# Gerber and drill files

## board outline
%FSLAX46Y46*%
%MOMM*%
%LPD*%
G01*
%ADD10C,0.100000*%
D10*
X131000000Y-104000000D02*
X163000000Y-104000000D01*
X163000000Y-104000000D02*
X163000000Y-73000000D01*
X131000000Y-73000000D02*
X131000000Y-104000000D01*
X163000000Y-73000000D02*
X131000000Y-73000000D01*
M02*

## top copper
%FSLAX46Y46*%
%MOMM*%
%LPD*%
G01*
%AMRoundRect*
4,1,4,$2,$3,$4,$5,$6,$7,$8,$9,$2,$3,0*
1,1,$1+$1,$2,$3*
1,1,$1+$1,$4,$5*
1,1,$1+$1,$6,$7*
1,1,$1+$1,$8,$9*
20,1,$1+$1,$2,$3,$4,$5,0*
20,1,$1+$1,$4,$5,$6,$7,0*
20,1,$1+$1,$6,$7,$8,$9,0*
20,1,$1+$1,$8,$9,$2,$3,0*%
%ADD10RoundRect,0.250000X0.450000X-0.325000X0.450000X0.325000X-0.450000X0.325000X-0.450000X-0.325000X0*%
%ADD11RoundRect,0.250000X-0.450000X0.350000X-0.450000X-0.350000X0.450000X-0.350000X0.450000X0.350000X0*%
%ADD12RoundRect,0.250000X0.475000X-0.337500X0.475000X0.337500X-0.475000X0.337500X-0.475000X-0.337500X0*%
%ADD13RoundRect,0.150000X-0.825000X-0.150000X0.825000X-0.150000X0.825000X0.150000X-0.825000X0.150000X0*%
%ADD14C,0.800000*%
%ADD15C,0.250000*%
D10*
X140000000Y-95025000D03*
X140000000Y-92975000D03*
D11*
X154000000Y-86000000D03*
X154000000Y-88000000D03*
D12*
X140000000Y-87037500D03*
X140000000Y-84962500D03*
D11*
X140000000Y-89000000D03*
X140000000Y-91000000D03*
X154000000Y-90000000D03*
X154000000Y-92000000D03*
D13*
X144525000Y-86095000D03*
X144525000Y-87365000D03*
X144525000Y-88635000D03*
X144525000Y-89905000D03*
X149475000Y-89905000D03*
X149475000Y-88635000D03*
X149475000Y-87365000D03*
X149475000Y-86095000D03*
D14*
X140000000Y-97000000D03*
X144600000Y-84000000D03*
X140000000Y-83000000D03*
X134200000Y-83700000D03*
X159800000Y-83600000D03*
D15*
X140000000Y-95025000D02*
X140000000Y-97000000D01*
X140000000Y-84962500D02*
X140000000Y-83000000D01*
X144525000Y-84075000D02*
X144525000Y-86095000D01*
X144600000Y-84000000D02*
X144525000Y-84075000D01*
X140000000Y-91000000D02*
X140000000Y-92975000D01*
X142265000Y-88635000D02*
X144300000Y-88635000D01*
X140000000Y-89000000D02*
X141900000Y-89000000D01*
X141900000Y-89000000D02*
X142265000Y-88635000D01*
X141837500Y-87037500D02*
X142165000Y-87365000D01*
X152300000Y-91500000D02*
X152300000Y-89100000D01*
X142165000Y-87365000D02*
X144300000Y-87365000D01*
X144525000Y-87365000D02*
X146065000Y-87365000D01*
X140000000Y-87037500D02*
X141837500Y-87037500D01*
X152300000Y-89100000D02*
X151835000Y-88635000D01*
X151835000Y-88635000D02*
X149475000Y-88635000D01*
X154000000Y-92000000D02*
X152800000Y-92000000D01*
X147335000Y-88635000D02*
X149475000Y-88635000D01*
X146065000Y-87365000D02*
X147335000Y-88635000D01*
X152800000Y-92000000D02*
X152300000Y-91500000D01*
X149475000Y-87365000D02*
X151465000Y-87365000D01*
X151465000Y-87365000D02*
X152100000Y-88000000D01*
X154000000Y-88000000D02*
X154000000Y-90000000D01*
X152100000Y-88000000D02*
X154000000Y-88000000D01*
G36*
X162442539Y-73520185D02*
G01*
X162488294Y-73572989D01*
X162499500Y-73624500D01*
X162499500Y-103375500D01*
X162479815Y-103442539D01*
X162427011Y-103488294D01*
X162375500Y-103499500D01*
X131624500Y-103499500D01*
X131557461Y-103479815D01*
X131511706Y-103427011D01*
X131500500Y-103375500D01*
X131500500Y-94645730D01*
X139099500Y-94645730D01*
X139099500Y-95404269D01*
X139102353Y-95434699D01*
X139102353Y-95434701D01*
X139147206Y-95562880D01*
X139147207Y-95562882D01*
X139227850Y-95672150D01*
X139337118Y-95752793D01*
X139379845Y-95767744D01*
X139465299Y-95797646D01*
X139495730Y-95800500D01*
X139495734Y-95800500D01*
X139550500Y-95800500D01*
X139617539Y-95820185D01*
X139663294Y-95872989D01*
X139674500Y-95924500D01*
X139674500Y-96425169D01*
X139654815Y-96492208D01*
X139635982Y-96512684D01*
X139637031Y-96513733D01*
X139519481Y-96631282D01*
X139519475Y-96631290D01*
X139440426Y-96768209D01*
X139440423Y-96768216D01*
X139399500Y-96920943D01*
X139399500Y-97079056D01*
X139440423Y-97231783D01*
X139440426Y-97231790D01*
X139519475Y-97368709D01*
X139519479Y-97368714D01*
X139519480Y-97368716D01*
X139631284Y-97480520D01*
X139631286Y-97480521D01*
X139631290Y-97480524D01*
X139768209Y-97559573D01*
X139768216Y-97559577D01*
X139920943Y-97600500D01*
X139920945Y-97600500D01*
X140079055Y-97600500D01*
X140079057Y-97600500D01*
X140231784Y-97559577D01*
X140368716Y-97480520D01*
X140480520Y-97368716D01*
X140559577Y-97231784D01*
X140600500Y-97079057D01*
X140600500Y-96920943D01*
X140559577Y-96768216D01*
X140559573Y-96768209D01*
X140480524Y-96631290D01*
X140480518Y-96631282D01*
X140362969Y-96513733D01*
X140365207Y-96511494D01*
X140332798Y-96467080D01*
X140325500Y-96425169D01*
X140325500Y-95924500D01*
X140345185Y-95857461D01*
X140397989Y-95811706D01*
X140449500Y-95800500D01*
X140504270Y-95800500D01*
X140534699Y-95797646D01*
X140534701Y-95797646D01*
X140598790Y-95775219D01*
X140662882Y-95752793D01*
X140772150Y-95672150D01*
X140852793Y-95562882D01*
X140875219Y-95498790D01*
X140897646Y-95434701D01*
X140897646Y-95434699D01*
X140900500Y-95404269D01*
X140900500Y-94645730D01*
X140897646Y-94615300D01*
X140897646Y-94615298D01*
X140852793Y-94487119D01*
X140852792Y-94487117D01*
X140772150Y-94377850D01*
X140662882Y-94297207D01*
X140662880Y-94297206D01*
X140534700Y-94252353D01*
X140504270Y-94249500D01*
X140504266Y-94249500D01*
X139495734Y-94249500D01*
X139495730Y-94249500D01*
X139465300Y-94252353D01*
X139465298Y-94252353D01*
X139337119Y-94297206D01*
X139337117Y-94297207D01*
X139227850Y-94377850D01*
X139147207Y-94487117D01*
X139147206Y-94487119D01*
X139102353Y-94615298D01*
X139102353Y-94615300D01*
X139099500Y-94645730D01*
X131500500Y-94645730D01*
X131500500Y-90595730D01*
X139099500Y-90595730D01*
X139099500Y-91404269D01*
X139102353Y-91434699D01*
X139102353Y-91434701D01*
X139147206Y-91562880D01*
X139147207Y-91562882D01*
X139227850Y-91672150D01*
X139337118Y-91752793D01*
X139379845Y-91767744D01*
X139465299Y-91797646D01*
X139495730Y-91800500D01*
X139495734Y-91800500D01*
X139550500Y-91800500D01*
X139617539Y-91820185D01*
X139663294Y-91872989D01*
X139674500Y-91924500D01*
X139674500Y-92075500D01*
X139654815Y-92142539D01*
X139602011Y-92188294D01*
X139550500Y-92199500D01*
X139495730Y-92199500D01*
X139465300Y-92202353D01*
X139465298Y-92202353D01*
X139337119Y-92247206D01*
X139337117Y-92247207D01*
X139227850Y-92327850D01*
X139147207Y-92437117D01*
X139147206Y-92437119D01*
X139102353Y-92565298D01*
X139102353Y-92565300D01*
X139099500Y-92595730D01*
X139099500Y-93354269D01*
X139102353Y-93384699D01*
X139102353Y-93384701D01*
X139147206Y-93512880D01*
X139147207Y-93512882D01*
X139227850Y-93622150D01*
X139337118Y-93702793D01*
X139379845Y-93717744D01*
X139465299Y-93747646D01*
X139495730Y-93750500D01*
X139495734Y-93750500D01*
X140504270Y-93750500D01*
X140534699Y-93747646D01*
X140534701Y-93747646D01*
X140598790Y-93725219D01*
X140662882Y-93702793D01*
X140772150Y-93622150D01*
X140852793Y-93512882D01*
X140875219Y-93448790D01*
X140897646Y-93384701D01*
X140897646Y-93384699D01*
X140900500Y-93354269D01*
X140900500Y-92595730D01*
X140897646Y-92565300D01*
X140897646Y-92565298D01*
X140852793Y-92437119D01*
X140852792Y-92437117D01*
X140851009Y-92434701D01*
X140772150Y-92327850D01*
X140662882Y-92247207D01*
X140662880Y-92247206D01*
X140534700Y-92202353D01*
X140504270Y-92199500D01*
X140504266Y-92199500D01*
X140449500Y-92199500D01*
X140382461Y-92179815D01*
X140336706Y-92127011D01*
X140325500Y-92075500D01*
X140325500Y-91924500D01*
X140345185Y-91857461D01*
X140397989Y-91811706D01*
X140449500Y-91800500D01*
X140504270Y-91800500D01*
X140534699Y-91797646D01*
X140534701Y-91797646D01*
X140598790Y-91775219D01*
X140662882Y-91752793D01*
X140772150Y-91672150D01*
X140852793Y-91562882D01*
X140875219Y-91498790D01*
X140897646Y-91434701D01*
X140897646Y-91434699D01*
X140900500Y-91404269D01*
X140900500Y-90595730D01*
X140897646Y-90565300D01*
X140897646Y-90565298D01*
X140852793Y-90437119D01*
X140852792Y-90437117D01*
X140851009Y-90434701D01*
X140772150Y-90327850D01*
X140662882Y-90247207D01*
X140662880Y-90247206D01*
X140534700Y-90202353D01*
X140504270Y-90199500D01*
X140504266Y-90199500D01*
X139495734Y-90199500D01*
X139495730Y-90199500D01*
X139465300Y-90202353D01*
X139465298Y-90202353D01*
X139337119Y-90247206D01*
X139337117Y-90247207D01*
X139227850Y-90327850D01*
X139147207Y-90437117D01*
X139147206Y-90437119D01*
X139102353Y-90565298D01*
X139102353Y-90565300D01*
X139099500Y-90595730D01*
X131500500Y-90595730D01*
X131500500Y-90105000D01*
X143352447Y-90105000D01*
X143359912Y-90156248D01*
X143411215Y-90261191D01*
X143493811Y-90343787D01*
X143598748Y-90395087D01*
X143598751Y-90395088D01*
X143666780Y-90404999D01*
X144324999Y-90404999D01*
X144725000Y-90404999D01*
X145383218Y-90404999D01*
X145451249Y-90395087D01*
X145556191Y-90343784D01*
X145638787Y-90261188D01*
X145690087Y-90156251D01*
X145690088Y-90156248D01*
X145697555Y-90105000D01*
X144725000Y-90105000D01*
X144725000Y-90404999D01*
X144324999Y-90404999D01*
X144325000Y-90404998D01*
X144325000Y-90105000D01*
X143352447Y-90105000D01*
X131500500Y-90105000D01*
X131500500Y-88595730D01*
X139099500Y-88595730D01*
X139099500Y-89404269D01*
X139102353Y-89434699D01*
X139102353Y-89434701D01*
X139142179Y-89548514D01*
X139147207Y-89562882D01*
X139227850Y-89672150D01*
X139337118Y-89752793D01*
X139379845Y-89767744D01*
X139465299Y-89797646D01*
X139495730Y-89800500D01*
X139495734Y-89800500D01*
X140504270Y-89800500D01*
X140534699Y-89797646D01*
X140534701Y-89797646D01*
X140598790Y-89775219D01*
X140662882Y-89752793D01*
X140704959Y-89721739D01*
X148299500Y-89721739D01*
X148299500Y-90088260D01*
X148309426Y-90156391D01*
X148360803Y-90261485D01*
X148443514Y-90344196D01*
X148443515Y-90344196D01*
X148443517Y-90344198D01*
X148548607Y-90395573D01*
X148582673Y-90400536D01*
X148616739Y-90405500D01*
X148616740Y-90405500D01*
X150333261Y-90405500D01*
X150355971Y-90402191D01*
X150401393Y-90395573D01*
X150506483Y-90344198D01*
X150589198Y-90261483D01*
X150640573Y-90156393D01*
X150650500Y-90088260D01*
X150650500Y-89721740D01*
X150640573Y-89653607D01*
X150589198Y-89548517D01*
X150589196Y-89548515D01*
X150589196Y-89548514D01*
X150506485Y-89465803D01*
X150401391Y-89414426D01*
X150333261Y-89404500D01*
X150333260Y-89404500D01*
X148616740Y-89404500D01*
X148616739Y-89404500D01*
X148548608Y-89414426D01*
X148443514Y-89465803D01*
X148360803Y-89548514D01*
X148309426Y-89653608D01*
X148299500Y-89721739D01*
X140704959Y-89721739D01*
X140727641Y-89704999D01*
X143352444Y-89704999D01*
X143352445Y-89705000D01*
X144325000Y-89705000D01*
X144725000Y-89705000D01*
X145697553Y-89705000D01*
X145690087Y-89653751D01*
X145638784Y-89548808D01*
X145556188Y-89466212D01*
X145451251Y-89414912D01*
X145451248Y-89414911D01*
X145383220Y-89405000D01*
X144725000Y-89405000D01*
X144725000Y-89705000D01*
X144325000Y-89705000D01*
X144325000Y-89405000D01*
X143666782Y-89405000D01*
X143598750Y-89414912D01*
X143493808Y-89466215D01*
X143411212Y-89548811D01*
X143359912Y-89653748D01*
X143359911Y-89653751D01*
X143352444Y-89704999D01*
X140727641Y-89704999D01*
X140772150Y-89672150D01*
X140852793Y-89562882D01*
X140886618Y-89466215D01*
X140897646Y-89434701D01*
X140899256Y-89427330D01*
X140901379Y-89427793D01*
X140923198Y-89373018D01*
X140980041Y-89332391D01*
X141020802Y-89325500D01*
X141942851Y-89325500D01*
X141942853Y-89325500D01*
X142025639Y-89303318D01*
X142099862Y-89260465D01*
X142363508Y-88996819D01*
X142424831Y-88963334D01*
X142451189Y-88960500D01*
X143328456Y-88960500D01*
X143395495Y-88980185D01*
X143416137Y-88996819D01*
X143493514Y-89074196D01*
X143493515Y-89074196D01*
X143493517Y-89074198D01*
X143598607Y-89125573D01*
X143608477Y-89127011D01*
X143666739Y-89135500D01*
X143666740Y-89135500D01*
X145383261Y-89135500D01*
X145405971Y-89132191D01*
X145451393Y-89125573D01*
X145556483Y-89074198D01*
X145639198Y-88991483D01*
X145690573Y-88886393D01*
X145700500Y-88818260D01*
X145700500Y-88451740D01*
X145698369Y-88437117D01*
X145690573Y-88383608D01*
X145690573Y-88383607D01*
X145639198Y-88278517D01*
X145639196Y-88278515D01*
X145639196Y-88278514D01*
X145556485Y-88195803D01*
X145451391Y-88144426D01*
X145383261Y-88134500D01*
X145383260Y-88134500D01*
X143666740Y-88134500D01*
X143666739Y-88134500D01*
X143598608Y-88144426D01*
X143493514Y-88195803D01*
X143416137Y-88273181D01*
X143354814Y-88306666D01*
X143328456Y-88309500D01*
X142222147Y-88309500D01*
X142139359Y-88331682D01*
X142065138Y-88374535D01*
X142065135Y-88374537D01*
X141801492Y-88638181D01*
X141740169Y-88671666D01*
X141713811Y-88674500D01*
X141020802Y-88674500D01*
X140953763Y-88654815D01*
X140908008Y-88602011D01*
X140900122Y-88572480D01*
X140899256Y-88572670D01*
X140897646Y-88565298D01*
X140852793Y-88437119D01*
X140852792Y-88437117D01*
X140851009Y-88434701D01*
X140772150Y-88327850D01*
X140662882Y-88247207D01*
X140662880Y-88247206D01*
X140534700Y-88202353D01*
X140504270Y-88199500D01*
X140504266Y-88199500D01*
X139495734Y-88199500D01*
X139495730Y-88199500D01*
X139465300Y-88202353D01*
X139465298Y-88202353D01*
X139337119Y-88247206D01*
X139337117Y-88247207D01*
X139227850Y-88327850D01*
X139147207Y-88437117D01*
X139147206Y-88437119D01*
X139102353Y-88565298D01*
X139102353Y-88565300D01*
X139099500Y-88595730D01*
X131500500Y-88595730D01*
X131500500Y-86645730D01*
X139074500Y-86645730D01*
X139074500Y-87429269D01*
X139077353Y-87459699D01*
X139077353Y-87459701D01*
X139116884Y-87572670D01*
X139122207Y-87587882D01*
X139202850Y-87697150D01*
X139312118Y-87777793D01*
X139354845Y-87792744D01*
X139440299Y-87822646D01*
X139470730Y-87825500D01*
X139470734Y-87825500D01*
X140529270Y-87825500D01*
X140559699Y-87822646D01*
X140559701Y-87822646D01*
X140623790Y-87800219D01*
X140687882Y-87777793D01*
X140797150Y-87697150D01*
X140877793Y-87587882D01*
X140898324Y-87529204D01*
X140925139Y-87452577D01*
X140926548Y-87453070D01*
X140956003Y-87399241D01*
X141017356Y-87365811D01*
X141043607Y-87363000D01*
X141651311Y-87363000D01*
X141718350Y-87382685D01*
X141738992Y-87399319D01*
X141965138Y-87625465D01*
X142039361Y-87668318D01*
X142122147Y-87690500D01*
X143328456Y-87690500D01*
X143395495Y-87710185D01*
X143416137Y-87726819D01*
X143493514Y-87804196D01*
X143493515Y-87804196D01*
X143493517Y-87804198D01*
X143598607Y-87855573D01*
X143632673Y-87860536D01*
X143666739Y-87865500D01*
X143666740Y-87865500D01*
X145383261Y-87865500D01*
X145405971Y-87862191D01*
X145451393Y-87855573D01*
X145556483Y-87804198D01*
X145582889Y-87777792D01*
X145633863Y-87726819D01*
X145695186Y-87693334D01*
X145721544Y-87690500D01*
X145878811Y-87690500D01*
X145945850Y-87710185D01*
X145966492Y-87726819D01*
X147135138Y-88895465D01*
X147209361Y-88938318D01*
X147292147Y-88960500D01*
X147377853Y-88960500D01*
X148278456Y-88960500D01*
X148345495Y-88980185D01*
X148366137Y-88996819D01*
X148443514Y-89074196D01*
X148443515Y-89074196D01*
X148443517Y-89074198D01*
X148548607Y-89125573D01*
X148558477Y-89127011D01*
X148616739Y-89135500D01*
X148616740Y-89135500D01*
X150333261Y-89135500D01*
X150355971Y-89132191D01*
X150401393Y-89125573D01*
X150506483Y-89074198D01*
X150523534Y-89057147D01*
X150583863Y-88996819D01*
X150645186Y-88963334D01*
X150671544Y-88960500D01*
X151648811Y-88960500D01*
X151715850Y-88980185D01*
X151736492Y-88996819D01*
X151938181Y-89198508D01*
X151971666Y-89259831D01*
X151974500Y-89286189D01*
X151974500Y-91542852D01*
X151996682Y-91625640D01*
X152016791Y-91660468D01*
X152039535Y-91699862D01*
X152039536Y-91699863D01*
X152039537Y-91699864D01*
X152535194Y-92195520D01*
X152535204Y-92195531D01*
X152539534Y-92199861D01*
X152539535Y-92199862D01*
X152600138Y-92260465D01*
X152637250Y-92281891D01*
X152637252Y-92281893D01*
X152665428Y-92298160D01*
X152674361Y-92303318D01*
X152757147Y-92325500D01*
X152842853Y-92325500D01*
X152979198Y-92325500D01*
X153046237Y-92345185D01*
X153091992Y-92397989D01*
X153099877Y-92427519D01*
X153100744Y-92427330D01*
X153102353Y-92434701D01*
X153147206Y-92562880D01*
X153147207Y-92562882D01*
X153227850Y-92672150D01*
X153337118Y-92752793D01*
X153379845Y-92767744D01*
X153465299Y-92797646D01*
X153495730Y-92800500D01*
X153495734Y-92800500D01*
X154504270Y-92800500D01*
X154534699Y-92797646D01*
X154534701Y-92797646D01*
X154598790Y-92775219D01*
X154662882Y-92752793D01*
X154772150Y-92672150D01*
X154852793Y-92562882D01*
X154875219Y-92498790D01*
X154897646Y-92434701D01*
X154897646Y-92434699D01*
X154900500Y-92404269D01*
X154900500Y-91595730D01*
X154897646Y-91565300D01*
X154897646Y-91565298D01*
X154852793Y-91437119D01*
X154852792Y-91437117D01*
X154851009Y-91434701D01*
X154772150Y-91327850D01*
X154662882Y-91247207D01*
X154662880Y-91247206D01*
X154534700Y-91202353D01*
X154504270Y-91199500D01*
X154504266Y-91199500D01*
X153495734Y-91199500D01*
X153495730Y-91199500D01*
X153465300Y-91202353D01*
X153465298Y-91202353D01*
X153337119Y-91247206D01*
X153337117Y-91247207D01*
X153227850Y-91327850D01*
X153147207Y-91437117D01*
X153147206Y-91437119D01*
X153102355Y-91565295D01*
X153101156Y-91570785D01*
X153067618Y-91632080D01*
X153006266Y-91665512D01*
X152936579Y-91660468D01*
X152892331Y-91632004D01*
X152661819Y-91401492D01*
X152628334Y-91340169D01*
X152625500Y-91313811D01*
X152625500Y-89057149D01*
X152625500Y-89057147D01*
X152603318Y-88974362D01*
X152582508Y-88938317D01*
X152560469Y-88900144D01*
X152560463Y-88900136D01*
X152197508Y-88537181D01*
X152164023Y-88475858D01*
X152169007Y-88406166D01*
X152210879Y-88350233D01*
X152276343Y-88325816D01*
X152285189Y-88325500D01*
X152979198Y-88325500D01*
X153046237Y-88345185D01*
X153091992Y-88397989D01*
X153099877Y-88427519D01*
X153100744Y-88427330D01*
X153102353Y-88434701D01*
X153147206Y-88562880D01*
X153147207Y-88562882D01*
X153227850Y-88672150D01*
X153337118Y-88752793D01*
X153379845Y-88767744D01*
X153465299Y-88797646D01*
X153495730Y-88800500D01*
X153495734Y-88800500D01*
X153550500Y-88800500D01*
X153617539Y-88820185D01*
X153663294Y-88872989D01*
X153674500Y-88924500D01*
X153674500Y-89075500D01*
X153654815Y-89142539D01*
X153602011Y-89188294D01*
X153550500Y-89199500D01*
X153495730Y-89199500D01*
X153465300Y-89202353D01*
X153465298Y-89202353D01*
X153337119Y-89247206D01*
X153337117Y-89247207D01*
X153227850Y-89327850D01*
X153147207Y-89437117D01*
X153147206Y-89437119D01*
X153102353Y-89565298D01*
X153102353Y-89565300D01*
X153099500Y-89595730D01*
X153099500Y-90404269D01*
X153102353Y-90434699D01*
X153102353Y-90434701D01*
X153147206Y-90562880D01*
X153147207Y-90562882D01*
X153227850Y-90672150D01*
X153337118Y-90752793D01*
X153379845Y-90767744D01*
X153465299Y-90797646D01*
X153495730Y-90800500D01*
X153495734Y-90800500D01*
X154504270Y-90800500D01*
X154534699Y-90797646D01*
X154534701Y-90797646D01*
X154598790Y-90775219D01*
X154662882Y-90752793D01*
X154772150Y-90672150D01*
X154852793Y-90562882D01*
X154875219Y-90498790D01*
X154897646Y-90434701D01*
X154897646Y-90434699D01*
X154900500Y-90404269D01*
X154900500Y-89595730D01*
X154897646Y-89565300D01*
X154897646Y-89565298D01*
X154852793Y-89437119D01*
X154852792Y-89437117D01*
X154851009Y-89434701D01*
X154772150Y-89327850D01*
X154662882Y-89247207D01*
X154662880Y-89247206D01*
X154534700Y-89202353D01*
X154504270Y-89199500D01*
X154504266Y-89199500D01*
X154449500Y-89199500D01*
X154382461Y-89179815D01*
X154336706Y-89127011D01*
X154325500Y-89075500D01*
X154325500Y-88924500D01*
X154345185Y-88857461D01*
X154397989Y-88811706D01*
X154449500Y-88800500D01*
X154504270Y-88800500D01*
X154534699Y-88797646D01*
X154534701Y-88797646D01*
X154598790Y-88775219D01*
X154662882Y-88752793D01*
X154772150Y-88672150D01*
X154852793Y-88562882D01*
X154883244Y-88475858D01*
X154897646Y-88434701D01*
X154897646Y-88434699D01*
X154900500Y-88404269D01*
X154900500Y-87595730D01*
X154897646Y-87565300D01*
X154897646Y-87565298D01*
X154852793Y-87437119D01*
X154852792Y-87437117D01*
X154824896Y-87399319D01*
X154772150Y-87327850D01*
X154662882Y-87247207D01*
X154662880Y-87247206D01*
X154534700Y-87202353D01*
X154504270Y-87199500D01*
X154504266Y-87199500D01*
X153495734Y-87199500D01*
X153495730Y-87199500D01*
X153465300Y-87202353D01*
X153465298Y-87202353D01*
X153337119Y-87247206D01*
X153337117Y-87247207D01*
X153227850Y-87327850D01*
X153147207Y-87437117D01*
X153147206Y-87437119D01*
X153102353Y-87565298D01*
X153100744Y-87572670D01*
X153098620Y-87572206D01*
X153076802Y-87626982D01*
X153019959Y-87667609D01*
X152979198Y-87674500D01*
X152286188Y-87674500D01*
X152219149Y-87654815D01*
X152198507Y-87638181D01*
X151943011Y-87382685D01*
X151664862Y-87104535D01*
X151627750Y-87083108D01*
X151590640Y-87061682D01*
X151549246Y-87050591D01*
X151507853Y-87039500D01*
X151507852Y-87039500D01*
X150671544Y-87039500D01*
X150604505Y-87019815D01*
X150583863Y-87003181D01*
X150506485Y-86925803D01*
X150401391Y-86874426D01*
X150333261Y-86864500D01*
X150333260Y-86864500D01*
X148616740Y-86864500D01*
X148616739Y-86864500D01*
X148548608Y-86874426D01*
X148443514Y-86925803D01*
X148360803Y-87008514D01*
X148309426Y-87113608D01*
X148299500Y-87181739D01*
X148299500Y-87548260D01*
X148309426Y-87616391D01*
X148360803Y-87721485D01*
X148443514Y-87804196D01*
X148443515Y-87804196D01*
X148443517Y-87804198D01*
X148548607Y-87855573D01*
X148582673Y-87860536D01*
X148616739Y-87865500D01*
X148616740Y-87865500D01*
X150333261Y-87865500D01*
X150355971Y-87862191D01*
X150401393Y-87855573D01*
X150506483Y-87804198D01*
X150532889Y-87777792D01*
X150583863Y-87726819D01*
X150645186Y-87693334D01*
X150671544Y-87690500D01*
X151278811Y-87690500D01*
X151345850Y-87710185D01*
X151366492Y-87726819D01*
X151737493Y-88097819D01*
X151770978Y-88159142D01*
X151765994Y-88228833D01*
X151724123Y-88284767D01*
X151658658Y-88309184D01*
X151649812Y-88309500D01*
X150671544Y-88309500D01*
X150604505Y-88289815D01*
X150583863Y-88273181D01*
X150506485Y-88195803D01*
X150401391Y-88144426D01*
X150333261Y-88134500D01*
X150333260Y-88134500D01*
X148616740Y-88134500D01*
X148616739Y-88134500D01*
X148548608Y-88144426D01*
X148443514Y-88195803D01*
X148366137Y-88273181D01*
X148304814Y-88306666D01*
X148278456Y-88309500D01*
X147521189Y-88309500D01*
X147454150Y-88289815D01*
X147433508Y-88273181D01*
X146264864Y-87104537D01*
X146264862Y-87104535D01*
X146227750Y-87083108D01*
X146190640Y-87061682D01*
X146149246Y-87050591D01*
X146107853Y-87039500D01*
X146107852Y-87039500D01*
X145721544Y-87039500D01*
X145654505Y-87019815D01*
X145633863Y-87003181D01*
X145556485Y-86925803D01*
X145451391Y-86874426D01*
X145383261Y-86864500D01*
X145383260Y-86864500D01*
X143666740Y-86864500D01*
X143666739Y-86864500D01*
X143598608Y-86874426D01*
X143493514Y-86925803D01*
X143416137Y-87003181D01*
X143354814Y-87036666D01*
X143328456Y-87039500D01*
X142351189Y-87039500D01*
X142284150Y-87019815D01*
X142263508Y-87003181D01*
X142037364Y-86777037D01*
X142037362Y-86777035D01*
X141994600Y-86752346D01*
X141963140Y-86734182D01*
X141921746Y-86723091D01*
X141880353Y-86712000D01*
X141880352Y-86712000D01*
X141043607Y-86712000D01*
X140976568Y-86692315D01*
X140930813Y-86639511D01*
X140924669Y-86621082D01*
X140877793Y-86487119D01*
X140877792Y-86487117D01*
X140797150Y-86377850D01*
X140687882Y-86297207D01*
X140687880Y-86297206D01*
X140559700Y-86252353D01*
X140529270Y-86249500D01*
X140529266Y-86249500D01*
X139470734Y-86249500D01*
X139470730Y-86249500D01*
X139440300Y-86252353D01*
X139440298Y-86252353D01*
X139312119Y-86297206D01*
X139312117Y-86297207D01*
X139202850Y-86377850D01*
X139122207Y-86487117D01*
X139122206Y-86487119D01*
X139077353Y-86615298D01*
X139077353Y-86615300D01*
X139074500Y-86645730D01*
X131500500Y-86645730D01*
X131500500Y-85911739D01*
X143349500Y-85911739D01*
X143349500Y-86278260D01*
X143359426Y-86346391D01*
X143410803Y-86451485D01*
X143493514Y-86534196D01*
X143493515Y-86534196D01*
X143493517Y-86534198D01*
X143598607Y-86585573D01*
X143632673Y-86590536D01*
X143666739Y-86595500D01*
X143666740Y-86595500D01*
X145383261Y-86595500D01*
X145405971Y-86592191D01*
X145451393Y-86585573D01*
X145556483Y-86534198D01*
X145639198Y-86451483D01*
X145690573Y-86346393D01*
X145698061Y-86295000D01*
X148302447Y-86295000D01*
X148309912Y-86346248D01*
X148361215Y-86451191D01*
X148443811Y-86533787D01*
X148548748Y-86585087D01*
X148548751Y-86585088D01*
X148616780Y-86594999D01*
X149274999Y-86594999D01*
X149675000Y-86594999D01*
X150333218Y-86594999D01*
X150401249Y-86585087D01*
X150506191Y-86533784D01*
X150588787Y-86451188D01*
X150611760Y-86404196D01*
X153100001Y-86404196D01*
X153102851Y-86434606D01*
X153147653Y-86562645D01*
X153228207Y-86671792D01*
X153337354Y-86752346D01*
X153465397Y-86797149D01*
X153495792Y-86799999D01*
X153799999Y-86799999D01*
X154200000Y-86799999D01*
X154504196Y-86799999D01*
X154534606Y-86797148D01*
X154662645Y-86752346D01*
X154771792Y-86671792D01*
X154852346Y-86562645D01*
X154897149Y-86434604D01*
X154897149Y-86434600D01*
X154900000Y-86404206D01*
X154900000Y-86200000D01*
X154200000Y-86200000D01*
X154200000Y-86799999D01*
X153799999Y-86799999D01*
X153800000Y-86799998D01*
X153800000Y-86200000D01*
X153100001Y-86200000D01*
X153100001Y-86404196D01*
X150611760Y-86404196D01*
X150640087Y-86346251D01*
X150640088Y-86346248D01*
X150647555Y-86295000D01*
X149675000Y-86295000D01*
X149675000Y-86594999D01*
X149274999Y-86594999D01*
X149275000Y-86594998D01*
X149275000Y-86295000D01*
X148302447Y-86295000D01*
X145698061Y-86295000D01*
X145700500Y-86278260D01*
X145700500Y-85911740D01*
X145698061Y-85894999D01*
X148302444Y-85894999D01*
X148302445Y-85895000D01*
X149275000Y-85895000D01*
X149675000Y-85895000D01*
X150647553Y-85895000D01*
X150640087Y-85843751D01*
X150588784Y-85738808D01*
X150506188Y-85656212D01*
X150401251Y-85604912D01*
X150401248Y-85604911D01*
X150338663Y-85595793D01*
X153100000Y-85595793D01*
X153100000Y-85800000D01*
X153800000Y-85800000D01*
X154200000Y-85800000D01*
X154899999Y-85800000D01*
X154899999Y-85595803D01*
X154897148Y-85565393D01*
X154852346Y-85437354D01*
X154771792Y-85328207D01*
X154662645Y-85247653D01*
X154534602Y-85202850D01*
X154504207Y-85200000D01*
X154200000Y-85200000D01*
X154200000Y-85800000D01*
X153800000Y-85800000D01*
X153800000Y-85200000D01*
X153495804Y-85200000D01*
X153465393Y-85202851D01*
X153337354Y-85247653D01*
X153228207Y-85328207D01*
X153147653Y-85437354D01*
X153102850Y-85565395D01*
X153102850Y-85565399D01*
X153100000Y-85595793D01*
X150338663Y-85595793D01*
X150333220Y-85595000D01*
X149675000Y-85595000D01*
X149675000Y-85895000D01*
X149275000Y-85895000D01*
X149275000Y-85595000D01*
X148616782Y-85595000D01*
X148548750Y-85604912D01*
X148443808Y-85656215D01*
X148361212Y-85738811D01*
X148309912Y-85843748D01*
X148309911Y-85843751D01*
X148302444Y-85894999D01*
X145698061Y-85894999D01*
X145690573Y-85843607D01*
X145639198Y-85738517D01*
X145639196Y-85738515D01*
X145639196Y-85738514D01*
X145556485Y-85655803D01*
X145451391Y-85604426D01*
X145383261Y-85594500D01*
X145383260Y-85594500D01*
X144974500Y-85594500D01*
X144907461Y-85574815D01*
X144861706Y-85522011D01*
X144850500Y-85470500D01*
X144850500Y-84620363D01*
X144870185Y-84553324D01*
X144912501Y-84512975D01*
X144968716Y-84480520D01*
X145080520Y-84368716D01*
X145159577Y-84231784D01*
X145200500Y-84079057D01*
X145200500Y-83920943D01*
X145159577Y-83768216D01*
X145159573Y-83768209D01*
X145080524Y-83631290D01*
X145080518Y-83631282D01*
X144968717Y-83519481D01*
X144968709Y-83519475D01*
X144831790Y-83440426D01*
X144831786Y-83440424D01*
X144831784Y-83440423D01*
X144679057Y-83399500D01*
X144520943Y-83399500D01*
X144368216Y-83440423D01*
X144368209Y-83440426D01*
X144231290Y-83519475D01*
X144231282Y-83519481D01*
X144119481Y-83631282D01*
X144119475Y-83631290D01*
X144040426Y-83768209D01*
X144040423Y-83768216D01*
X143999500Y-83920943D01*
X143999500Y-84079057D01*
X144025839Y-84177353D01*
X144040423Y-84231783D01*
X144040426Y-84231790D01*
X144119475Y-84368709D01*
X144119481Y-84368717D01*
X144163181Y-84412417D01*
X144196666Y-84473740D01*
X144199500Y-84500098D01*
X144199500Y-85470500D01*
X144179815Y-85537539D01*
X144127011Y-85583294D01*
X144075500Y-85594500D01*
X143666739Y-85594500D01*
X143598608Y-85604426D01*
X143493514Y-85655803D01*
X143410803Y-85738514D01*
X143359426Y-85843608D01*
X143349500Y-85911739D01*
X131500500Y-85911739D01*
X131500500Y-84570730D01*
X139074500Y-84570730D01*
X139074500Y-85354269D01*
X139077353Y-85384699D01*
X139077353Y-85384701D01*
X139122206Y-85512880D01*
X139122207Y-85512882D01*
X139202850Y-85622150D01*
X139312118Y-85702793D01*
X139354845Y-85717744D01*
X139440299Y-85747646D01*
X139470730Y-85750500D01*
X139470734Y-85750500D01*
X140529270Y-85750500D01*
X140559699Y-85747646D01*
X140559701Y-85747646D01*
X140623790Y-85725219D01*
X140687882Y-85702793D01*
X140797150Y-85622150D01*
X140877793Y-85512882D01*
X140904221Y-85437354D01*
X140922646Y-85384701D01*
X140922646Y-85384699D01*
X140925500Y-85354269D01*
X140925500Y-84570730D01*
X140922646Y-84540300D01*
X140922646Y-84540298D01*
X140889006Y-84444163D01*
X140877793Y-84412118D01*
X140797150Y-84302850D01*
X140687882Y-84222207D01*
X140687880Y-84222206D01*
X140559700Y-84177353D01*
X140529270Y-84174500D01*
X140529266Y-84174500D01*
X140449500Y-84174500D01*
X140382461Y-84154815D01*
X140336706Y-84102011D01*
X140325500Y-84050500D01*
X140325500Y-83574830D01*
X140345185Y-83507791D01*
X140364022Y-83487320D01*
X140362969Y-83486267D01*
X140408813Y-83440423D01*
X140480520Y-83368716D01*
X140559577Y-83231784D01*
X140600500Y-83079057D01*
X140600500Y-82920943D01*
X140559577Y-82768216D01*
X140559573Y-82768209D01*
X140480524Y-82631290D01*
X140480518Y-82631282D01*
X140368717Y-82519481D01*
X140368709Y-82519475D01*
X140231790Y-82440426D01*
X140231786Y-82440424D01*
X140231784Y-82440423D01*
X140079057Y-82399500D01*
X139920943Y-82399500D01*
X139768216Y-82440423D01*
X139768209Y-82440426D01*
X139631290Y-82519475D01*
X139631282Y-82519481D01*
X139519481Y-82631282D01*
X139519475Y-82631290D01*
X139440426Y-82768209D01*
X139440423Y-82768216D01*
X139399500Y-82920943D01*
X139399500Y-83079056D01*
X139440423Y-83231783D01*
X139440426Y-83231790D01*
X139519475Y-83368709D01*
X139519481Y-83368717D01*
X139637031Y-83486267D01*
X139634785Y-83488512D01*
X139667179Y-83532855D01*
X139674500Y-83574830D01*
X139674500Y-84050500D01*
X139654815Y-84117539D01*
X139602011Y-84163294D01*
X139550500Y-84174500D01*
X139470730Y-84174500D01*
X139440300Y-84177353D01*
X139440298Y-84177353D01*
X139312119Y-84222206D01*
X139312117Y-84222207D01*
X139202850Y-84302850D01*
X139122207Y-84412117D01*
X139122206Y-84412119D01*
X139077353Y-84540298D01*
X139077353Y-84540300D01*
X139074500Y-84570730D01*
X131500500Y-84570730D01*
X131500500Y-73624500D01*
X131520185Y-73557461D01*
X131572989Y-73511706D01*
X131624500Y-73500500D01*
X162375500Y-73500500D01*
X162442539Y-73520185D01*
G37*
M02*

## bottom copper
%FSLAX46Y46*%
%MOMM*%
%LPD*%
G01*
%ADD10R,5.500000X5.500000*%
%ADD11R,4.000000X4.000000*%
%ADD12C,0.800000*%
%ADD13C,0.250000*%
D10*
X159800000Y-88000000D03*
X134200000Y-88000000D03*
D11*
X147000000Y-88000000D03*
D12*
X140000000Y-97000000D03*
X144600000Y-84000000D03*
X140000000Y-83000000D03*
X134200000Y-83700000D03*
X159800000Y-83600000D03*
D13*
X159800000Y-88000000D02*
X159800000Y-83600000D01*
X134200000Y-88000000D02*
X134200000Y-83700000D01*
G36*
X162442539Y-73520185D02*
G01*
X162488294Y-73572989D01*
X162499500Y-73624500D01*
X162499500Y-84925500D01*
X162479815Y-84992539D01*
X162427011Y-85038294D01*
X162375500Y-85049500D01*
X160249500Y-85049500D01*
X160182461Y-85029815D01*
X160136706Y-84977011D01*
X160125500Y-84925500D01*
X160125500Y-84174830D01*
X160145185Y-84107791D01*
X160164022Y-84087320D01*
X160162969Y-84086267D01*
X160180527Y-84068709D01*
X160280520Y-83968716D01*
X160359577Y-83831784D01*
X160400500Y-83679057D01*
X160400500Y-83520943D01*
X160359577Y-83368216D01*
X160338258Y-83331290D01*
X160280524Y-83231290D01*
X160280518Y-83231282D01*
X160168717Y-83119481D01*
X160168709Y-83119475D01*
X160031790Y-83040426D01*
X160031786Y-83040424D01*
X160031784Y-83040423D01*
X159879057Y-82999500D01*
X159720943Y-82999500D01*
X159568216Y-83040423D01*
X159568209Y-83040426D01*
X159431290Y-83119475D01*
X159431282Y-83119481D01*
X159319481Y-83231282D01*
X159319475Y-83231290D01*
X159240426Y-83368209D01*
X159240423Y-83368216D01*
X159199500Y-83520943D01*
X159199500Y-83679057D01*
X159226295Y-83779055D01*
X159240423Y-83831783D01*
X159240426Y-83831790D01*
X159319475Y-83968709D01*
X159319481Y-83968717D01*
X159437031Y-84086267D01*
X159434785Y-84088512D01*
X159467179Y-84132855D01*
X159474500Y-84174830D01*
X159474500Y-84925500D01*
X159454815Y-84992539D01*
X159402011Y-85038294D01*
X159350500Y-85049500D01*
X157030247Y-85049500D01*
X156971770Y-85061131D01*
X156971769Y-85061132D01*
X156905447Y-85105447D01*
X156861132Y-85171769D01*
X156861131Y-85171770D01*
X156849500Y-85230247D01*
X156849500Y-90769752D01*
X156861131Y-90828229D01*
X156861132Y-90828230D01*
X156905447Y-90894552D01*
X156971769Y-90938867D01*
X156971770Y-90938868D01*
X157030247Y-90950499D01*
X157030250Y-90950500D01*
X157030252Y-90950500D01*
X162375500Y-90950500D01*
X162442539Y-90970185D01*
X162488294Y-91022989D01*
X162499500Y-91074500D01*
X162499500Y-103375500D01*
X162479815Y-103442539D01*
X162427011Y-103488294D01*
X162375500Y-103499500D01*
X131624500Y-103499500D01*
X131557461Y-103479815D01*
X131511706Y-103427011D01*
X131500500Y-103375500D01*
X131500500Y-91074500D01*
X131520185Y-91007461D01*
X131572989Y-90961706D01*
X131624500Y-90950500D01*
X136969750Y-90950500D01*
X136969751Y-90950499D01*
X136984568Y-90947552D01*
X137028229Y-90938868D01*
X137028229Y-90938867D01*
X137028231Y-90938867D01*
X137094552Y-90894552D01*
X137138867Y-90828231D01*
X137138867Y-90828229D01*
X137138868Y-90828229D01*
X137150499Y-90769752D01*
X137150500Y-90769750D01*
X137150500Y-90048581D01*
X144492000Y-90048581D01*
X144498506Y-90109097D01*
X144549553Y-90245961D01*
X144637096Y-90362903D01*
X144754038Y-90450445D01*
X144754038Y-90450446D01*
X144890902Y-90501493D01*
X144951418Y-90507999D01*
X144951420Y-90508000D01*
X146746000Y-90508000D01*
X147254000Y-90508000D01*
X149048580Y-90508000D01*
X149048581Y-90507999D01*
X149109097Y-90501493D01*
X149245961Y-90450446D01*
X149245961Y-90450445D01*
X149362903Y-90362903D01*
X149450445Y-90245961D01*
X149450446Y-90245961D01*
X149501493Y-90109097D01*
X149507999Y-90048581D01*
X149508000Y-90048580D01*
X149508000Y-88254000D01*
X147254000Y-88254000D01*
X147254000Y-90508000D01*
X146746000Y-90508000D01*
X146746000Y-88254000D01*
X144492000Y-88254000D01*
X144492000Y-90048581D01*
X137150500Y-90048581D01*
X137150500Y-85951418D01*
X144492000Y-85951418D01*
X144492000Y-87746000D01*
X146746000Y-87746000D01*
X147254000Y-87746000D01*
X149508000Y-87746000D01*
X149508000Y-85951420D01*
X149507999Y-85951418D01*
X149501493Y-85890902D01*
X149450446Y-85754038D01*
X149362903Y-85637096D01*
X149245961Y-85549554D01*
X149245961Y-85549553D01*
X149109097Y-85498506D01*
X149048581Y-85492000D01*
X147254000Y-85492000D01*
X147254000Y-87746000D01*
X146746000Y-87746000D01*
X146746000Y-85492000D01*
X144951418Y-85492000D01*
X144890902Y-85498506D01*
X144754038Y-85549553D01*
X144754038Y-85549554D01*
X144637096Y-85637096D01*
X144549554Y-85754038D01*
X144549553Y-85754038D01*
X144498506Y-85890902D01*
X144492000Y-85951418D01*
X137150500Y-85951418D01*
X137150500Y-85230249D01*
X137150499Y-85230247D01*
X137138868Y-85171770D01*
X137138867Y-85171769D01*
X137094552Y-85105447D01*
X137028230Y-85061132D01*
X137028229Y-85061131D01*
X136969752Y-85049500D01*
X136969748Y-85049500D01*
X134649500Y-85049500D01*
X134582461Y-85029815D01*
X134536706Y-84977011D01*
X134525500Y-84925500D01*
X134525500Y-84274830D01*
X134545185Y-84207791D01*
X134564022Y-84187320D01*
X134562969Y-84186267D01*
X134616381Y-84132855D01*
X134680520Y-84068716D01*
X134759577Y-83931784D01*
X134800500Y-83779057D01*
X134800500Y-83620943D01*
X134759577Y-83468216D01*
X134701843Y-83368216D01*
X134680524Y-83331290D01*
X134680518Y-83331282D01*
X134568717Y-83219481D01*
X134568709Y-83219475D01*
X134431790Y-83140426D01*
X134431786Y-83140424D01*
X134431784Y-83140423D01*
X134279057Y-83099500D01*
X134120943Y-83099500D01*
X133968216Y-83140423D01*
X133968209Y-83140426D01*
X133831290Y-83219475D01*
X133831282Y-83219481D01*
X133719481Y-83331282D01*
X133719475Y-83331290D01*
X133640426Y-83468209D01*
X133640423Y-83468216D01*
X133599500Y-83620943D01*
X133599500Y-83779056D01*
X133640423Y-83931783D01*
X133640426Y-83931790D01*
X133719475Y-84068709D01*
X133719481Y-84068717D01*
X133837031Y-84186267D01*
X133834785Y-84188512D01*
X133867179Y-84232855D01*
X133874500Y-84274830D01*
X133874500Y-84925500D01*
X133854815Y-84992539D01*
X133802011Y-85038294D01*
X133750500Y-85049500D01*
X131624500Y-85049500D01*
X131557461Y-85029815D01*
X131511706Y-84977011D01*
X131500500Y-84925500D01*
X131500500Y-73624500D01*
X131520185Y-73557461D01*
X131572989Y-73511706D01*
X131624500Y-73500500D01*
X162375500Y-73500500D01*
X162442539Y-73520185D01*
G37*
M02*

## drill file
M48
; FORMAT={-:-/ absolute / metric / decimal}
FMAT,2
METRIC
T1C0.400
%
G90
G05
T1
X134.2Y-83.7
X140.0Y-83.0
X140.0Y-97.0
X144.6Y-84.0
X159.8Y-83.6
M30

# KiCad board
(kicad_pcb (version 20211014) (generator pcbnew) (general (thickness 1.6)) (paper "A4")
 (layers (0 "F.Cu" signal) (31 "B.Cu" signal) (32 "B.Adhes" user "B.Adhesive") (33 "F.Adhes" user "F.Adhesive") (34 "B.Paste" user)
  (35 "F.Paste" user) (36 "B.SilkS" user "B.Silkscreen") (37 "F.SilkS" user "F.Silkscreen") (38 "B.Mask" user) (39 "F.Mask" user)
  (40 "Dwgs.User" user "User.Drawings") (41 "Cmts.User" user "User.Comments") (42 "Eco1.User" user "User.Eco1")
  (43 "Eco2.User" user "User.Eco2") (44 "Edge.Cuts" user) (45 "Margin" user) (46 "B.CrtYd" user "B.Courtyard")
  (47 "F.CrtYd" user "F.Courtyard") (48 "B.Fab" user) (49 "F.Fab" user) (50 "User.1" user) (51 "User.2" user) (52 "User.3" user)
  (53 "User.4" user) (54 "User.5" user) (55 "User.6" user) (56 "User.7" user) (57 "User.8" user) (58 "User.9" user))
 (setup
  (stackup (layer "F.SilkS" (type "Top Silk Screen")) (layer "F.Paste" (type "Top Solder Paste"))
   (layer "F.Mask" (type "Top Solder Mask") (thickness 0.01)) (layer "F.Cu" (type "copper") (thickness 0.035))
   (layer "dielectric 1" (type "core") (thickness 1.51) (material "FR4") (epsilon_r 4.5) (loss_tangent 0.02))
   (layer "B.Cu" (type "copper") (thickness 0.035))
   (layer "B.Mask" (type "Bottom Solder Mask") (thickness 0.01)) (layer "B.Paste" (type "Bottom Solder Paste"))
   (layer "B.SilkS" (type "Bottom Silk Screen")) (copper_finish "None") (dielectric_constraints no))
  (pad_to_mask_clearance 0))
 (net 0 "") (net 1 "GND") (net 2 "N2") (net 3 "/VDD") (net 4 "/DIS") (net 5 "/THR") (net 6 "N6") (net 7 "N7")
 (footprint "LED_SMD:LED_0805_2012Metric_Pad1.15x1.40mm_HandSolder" (layer "F.Cu") (at 140 94 90)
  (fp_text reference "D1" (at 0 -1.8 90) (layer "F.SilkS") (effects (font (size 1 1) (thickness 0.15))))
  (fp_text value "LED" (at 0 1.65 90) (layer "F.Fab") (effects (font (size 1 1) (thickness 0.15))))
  (pad "1" smd roundrect (at -1.025 0 90) (size 1.15 1.4) (layers "F.Cu" "F.Paste" "F.Mask") (roundrect_rratio 0.2173913043) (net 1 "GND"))
  (pad "2" smd roundrect (at 1.025 0 90) (size 1.15 1.4) (layers "F.Cu" "F.Paste" "F.Mask") (roundrect_rratio 0.2173913043) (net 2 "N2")))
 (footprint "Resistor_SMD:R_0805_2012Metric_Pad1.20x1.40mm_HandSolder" (layer "F.Cu") (at 154 87 -90)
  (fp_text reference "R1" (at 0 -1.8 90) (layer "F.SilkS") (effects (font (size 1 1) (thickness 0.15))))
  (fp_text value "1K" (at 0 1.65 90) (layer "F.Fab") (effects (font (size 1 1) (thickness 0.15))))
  (pad "1" smd roundrect (at -1 0 270) (size 1.2 1.4) (layers "F.Cu" "F.Paste" "F.Mask") (roundrect_rratio 0.2083333333) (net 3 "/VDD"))
  (pad "2" smd roundrect (at 1 0 270) (size 1.2 1.4) (layers "F.Cu" "F.Paste" "F.Mask") (roundrect_rratio 0.2083333333) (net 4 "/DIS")))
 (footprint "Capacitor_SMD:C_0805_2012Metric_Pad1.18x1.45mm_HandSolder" (layer "F.Cu") (at 140 86 90)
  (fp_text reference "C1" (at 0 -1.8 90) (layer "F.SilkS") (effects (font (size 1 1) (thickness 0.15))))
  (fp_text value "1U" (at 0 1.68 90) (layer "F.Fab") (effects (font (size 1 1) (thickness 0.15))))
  (pad "1" smd roundrect (at -1.0375 0 90) (size 1.175 1.45) (layers "F.Cu" "F.Paste" "F.Mask") (roundrect_rratio 0.2127659574)
   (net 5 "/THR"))
  (pad "2" smd roundrect (at 1.0375 0 90) (size 1.175 1.45) (layers "F.Cu" "F.Paste" "F.Mask") (roundrect_rratio 0.2127659574) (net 1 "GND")))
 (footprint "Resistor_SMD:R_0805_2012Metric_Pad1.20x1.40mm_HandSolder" (layer "F.Cu") (at 140 90 -90)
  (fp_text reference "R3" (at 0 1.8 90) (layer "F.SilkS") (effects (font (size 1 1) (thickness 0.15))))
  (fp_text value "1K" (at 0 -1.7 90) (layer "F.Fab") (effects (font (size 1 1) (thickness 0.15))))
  (pad "1" smd roundrect (at -1 0 270) (size 1.2 1.4) (layers "F.Cu" "F.Paste" "F.Mask") (roundrect_rratio 0.2083333333) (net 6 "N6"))
  (pad "2" smd roundrect (at 1 0 270) (size 1.2 1.4) (layers "F.Cu" "F.Paste" "F.Mask") (roundrect_rratio 0.2083333333) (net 2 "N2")))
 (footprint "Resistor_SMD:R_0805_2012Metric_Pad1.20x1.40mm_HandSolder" (layer "F.Cu") (at 154 91 -90)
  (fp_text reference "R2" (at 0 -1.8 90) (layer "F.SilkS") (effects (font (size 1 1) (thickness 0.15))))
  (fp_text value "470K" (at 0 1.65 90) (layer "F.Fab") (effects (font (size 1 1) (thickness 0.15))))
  (pad "1" smd roundrect (at -1 0 270) (size 1.2 1.4) (layers "F.Cu" "F.Paste" "F.Mask") (roundrect_rratio 0.2083333333) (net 4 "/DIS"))
  (pad "2" smd roundrect (at 1 0 270) (size 1.2 1.4) (layers "F.Cu" "F.Paste" "F.Mask") (roundrect_rratio 0.2083333333) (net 5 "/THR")))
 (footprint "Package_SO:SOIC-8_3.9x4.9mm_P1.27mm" (layer "F.Cu") (at 147 88)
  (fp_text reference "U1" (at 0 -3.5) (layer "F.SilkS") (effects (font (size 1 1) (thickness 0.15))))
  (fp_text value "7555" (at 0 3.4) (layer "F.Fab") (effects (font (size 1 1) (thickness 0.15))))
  (pad "1" smd roundrect (at -2.475 -1.905) (size 1.95 0.6) (layers "F.Cu" "F.Paste" "F.Mask") (roundrect_rratio 0.25) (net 1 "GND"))
  (pad "2" smd roundrect (at -2.475 -0.635) (size 1.95 0.6) (layers "F.Cu" "F.Paste" "F.Mask") (roundrect_rratio 0.25) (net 5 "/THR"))
  (pad "3" smd roundrect (at -2.475 0.635) (size 1.95 0.6) (layers "F.Cu" "F.Paste" "F.Mask") (roundrect_rratio 0.25) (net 6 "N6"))
  (pad "4" smd roundrect (at -2.475 1.905) (size 1.95 0.6) (layers "F.Cu" "F.Paste" "F.Mask") (roundrect_rratio 0.25) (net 3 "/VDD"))
  (pad "5" smd roundrect (at 2.475 1.905) (size 1.95 0.6) (layers "F.Cu" "F.Paste" "F.Mask") (roundrect_rratio 0.25) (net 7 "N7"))
  (pad "6" smd roundrect (at 2.475 0.635) (size 1.95 0.6) (layers "F.Cu" "F.Paste" "F.Mask") (roundrect_rratio 0.25) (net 5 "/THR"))
  (pad "7" smd roundrect (at 2.475 -0.635) (size 1.95 0.6) (layers "F.Cu" "F.Paste" "F.Mask") (roundrect_rratio 0.25) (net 4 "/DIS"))
  (pad "8" smd roundrect (at 2.475 -1.905) (size 1.95 0.6) (layers "F.Cu" "F.Paste" "F.Mask") (roundrect_rratio 0.25) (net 3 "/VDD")))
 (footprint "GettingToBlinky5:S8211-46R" (layer "B.Cu") (at 147 88 180)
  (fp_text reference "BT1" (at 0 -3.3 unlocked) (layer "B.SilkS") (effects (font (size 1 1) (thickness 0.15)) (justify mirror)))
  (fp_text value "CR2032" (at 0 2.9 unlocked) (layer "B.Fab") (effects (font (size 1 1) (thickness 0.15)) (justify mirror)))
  (pad "1" smd rect (at -12.8 0 180) (size 5.5 5.5) (layers "B.Cu" "B.Paste" "B.Mask") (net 3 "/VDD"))
  (pad "1" smd rect (at 12.8 0 180) (size 5.5 5.5) (layers "B.Cu" "B.Paste" "B.Mask") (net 3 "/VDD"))
  (pad "2" smd rect (at 0 0 180) (size 4 4) (layers "B.Cu" "B.Paste" "B.Mask") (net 1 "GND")))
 (gr_line (start 131 104) (end 163 104) (layer "Edge.Cuts") (width 0.1))
 (gr_line (start 163 104) (end 163 73) (layer "Edge.Cuts") (width 0.1))
 (gr_line (start 131 73) (end 131 104) (layer "Edge.Cuts") (width 0.1))
 (gr_line (start 163 73) (end 131 73) (layer "Edge.Cuts") (width 0.1))
 (segment (start 140 95.025) (end 140 97) (width 0.25) (layer "F.Cu") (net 1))
 (segment (start 140 84.9625) (end 140 83) (width 0.25) (layer "F.Cu") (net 1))
 (segment (start 144.525 84.075) (end 144.525 86.095) (width 0.25) (layer "F.Cu") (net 1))
 (segment (start 144.6 84) (end 144.525 84.075) (width 0.25) (layer "F.Cu") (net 1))
 (via (at 140 97) (size 0.8) (drill 0.4) (layers "F.Cu" "B.Cu") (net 1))
 (via (at 144.6 84) (size 0.8) (drill 0.4) (layers "F.Cu" "B.Cu") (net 1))
 (via (at 140 83) (size 0.8) (drill 0.4) (layers "F.Cu" "B.Cu") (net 1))
 (segment (start 140 91) (end 140 92.975) (width 0.25) (layer "F.Cu") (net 2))
 (segment (start 142.265 88.635) (end 144.3 88.635) (width 0.25) (layer "F.Cu") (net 6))
 (segment (start 140 89) (end 141.9 89) (width 0.25) (layer "F.Cu") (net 6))
 (segment (start 141.9 89) (end 142.265 88.635) (width 0.25) (layer "F.Cu") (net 6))
 (via (at 134.2 83.7) (size 0.8) (drill 0.4) (layers "F.Cu" "B.Cu") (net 3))
 (via (at 159.8 83.6) (size 0.8) (drill 0.4) (layers "F.Cu" "B.Cu") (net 3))
 (segment (start 159.8 88) (end 159.8 83.6) (width 0.25) (layer "B.Cu") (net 3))
 (segment (start 134.2 88) (end 134.2 83.7) (width 0.25) (layer "B.Cu") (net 3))
 (segment (start 141.8375 87.0375) (end 142.165 87.365) (width 0.25) (layer "F.Cu") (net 5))
 (segment (start 152.3 91.5) (end 152.3 89.1) (width 0.25) (layer "F.Cu") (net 5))
 (segment (start 142.165 87.365) (end 144.3 87.365) (width 0.25) (layer "F.Cu") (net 5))
 (segment (start 144.525 87.365) (end 146.065 87.365) (width 0.25) (layer "F.Cu") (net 5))
 (segment (start 140 87.0375) (end 141.8375 87.0375) (width 0.25) (layer "F.Cu") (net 5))
 (segment (start 152.3 89.1) (end 151.835 88.635) (width 0.25) (layer "F.Cu") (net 5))
 (segment (start 151.835 88.635) (end 149.475 88.635) (width 0.25) (layer "F.Cu") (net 5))
 (segment (start 154 92) (end 152.8 92) (width 0.25) (layer "F.Cu") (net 5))
 (segment (start 147.335 88.635) (end 149.475 88.635) (width 0.25) (layer "F.Cu") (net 5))
 (segment (start 146.065 87.365) (end 147.335 88.635) (width 0.25) (layer "F.Cu") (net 5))
 (segment (start 152.8 92) (end 152.3 91.5) (width 0.25) (layer "F.Cu") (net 5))
 (segment (start 149.475 87.365) (end 151.465 87.365) (width 0.25) (layer "F.Cu") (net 4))
 (segment (start 151.465 87.365) (end 152.1 88) (width 0.25) (layer "F.Cu") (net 4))
 (segment (start 154 88) (end 154 90) (width 0.25) (layer "F.Cu") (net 4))
 (segment (start 152.1 88) (end 154 88) (width 0.25) (layer "F.Cu") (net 4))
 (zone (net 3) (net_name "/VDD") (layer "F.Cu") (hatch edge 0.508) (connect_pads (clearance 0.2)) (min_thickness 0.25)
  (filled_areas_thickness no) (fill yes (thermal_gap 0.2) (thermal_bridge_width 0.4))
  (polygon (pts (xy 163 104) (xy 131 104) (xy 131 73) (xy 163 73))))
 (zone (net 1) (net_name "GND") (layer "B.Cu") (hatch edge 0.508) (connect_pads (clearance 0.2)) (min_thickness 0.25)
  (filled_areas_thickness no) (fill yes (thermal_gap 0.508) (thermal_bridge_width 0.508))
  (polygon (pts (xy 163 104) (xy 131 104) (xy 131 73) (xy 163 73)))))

